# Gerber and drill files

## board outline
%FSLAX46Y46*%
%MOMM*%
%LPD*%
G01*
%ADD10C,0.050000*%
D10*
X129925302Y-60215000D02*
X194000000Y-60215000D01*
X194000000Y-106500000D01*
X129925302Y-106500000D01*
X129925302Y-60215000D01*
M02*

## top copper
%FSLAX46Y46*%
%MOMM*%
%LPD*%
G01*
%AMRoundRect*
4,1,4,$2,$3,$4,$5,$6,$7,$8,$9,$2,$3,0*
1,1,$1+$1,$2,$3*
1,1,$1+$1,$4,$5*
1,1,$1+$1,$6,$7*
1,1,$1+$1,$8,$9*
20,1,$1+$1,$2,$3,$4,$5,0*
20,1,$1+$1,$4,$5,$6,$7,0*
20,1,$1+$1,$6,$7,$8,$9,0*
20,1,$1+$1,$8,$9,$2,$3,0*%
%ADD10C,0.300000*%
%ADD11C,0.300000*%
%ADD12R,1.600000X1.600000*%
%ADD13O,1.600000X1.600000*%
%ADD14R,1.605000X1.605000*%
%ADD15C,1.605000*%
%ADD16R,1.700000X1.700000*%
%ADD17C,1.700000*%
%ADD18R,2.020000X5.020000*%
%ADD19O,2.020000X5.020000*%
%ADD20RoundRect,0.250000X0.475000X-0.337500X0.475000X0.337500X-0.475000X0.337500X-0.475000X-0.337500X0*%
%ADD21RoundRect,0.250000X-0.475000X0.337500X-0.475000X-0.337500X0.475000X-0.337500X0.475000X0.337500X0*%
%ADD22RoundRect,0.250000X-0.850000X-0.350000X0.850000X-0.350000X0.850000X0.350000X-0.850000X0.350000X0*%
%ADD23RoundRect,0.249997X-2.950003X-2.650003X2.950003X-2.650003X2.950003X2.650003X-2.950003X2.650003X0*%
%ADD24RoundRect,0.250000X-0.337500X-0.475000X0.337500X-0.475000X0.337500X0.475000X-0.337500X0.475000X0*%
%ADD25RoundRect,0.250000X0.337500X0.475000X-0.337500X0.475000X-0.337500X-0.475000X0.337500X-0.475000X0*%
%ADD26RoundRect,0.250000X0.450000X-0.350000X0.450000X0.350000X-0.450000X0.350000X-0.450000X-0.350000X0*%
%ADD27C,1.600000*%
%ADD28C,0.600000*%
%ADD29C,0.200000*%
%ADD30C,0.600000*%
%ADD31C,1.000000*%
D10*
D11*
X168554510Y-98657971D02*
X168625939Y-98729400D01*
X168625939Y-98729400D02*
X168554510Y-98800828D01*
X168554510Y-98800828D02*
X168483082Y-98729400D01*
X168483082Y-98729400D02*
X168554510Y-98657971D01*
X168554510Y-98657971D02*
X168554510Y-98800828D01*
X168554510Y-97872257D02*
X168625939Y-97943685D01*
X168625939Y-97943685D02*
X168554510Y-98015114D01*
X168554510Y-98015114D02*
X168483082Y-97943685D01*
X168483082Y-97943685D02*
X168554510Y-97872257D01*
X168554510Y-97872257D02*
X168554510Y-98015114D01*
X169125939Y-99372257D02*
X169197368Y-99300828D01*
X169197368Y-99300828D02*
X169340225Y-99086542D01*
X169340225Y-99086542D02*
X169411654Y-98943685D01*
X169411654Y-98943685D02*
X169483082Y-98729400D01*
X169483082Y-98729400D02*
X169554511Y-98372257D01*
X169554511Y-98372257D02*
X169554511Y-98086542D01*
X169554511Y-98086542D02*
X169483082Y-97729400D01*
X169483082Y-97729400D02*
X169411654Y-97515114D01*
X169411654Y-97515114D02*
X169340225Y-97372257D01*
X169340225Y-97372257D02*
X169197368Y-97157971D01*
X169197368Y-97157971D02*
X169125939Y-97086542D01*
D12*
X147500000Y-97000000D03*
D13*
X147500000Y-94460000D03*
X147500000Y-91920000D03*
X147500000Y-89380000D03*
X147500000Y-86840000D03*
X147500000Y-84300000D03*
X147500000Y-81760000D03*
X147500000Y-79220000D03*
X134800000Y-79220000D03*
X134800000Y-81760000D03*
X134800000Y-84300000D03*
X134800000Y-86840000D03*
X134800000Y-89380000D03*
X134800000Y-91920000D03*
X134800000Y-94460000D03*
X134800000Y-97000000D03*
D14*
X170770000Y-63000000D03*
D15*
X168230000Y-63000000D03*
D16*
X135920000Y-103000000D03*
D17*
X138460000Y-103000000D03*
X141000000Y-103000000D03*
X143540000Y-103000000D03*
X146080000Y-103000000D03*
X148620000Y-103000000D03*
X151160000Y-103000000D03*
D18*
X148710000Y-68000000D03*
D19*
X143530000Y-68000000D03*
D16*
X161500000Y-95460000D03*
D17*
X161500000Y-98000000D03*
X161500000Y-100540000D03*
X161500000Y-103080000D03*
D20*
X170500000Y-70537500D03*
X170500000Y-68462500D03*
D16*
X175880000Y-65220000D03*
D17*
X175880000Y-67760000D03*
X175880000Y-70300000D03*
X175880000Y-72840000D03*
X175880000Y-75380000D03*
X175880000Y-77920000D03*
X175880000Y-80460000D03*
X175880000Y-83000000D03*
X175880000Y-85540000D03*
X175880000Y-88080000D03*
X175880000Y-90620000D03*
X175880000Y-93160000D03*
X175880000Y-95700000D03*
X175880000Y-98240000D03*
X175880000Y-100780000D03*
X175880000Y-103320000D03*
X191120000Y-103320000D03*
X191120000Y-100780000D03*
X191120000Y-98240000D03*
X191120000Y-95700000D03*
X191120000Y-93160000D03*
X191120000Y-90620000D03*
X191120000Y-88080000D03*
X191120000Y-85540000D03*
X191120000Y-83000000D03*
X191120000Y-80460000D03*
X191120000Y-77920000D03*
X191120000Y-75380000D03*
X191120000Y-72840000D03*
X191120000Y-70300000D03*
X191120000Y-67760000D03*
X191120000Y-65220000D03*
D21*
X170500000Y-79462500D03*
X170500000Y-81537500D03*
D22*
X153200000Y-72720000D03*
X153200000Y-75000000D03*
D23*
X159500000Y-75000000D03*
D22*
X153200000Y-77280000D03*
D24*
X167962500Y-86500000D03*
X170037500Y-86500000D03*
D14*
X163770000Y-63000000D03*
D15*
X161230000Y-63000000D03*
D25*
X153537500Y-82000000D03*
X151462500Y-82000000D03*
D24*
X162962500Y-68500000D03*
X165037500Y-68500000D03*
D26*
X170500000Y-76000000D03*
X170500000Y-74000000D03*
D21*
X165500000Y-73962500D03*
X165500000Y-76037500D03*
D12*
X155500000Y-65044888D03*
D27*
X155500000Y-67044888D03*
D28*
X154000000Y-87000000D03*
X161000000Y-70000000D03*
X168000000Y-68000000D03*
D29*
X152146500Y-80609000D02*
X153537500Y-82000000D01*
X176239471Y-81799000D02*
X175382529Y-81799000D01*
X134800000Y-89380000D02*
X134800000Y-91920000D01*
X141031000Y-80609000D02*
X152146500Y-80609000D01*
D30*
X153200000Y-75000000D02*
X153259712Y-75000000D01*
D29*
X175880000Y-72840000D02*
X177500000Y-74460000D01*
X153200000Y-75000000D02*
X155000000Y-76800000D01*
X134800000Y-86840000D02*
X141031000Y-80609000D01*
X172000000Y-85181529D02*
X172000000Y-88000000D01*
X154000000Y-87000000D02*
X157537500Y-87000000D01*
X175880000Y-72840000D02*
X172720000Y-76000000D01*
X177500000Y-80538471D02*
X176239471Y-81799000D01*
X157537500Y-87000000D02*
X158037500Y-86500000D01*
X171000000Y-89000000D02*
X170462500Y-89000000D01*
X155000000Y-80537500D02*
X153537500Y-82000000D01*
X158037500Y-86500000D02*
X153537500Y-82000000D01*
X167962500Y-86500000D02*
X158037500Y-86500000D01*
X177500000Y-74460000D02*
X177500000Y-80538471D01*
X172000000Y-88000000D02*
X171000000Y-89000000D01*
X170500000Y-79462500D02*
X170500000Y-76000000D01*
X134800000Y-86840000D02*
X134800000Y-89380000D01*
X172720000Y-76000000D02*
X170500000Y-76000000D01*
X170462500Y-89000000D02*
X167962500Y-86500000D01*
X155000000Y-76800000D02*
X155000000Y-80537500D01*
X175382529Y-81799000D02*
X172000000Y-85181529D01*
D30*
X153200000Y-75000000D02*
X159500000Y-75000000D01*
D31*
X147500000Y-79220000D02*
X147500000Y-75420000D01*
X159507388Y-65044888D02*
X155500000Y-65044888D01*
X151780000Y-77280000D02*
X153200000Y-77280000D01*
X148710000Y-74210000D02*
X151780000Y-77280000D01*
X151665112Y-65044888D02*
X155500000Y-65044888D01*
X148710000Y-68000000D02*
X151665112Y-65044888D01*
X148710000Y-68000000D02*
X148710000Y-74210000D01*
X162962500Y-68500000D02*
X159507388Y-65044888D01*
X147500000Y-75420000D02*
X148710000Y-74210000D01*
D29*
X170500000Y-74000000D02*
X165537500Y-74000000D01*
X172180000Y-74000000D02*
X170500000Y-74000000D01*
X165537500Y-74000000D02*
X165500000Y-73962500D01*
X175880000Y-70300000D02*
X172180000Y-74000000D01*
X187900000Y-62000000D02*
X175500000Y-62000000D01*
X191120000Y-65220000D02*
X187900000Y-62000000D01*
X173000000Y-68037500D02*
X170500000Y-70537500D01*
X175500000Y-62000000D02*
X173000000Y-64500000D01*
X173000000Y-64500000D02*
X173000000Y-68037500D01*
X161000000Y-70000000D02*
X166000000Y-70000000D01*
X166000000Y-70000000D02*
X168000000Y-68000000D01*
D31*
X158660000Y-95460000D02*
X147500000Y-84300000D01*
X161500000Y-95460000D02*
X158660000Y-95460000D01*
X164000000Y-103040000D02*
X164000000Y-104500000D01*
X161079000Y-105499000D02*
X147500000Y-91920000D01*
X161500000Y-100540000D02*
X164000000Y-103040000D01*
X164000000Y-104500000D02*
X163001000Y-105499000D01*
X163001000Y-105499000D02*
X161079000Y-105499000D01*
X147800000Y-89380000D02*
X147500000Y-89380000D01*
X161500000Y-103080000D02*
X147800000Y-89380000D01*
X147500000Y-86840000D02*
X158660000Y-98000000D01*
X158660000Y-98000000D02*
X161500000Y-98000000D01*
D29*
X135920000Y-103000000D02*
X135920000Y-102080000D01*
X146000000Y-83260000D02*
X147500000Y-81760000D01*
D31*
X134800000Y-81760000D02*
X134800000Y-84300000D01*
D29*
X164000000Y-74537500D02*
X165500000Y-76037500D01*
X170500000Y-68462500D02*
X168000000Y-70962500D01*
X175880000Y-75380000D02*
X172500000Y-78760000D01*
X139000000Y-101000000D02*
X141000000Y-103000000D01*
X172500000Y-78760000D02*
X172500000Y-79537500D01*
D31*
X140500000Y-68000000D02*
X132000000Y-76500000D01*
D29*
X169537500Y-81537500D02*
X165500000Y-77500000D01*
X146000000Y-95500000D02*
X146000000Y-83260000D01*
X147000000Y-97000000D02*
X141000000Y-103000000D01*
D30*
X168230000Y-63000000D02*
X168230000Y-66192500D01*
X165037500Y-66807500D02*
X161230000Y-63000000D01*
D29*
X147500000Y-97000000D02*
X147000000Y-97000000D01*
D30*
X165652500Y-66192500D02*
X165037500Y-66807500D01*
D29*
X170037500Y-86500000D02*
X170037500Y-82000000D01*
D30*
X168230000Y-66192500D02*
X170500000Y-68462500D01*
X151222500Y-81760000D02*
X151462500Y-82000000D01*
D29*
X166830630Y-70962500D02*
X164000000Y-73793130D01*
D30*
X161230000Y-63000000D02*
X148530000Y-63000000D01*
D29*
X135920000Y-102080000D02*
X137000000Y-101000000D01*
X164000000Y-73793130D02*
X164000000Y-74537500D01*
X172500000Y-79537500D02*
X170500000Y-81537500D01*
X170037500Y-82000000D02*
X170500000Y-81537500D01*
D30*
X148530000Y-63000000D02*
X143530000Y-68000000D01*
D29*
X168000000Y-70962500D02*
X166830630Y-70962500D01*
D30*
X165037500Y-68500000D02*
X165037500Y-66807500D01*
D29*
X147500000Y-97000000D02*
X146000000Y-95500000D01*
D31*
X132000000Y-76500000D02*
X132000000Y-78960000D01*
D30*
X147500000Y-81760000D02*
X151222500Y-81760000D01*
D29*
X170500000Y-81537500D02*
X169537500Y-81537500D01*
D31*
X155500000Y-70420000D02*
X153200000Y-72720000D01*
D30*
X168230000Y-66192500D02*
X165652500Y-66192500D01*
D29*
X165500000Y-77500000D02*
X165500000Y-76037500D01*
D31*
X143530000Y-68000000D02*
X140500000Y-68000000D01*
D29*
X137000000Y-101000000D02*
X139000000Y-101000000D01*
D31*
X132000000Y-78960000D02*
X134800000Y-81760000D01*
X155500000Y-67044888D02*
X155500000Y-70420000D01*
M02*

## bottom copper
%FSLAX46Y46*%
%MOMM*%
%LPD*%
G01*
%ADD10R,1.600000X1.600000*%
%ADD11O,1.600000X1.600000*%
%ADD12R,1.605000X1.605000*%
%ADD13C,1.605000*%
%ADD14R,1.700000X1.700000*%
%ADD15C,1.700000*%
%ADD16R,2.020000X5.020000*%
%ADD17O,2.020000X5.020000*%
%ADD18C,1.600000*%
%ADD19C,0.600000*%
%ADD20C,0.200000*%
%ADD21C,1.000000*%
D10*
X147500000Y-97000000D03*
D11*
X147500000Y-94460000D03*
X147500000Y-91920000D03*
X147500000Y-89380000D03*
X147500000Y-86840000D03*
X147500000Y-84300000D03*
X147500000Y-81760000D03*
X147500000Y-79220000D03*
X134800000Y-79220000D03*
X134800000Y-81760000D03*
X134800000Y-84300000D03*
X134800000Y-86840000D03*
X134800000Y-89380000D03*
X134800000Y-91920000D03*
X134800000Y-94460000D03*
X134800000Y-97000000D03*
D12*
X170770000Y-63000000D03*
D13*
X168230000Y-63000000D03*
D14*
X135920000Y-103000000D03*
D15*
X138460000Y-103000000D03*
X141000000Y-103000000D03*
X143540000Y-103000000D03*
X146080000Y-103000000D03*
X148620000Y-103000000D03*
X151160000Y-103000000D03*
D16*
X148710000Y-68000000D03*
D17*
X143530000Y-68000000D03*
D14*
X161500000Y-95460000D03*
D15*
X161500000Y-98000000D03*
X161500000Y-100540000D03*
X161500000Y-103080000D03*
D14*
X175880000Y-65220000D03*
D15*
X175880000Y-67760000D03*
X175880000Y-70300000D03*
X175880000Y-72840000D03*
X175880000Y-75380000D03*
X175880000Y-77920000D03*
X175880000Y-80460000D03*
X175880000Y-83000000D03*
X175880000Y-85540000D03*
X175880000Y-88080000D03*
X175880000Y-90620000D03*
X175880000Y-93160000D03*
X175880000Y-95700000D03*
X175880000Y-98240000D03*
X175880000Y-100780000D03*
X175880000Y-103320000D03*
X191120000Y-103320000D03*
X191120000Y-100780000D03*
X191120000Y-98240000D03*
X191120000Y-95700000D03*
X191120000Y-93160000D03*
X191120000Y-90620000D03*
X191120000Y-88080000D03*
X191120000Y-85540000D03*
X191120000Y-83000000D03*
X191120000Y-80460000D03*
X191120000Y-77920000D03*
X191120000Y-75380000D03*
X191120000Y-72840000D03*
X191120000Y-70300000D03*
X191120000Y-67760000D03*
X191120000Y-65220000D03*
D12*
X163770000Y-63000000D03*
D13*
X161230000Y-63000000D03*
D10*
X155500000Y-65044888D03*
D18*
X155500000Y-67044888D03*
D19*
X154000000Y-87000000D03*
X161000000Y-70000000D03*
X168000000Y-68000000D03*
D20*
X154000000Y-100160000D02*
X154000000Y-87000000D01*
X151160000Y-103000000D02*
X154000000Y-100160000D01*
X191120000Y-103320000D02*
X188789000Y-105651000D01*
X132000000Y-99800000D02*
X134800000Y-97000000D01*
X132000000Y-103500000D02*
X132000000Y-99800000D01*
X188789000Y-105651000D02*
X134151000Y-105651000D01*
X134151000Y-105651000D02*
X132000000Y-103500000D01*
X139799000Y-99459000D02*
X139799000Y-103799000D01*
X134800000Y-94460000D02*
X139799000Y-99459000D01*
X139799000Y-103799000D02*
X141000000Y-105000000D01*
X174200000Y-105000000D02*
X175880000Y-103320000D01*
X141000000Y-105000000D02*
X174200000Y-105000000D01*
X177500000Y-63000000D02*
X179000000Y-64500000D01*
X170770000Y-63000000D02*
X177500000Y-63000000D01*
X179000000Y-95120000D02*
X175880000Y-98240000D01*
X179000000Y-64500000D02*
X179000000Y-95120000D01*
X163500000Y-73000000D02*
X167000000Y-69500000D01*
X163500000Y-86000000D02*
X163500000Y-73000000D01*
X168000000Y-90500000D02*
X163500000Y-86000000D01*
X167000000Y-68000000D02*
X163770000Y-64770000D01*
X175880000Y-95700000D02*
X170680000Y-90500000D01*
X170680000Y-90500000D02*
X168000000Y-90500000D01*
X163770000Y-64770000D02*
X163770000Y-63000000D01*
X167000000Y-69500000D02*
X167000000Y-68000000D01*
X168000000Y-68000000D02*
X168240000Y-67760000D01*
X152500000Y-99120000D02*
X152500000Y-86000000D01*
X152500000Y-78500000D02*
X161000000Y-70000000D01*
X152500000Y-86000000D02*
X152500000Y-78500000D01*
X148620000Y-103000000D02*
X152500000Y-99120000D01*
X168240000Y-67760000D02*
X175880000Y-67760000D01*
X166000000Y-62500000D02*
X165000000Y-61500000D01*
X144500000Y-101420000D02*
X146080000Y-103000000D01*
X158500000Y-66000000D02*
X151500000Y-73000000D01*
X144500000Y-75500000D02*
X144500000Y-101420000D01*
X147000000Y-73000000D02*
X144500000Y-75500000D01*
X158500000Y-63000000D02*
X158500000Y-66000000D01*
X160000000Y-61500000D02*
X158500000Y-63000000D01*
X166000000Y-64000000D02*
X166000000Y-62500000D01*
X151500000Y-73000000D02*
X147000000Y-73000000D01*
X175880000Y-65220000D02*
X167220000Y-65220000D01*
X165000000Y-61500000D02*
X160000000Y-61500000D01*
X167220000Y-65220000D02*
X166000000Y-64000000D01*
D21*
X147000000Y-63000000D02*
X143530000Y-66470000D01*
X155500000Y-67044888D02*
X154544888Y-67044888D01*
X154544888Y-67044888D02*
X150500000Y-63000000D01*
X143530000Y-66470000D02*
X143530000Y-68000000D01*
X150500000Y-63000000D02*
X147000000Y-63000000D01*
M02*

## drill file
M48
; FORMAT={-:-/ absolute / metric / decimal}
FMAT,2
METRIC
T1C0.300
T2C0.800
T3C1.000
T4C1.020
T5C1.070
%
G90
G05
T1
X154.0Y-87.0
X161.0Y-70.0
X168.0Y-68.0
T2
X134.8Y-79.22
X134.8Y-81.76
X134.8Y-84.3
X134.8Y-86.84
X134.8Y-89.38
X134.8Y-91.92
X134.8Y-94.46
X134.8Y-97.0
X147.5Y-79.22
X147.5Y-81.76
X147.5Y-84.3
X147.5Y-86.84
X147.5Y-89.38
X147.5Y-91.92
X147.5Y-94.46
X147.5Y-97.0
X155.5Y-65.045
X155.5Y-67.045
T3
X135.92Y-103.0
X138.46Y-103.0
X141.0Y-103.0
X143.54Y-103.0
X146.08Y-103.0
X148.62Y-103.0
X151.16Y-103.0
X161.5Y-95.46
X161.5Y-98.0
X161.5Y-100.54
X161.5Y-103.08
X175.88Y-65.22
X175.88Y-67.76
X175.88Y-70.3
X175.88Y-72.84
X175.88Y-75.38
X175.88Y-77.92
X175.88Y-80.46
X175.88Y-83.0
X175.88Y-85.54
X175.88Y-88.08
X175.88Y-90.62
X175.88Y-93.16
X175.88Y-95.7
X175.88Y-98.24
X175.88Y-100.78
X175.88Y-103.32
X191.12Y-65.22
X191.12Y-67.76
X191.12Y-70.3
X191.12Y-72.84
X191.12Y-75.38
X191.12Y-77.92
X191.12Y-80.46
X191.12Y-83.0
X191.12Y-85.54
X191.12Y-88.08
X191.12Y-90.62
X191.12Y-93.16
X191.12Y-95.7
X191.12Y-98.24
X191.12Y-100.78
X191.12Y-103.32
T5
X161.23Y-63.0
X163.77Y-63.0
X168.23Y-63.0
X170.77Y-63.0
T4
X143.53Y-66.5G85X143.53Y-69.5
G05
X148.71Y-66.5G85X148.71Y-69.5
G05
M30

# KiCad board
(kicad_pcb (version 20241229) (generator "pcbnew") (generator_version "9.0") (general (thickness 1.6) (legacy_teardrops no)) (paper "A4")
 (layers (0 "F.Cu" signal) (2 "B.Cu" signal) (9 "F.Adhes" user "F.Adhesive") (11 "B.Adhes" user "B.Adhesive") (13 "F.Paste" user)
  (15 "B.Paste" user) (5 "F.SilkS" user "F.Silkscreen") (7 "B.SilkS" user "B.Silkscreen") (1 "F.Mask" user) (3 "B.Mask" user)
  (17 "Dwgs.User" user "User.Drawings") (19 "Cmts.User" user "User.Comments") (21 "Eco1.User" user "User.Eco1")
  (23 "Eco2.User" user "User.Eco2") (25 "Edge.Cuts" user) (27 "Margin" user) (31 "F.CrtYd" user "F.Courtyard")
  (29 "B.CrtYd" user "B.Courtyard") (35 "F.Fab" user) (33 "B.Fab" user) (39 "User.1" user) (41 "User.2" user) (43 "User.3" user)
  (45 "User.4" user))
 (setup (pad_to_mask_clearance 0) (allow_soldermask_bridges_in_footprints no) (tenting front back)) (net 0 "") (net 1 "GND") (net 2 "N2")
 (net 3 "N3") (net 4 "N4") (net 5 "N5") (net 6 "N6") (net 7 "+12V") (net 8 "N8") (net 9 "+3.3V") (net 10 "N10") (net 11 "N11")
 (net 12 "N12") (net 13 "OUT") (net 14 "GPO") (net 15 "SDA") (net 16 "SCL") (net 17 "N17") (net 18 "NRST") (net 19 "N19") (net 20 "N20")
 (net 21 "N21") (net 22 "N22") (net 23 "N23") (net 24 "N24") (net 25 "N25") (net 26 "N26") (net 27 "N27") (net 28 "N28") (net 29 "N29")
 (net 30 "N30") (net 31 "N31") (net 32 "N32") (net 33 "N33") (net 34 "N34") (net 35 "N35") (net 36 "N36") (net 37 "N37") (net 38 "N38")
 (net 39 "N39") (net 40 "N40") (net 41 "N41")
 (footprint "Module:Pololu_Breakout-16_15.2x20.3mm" (layer "F.Cu") (at 147.5 97 180)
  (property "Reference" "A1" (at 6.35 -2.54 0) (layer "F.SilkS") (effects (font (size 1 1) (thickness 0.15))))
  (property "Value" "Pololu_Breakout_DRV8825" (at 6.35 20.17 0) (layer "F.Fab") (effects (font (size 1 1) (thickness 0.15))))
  (pad "1" thru_hole rect (at 0 0 180) (size 1.6 1.6) (drill 0.8) (layers "*.Cu" "*.Mask") (remove_unused_layers no) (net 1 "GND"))
  (pad "2" thru_hole oval (at 0 2.54 180) (size 1.6 1.6) (drill 0.8) (layers "*.Cu" "*.Mask") (remove_unused_layers no) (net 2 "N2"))
  (pad "3" thru_hole oval (at 0 5.08 180) (size 1.6 1.6) (drill 0.8) (layers "*.Cu" "*.Mask") (remove_unused_layers no) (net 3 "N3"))
  (pad "4" thru_hole oval (at 0 7.62 180) (size 1.6 1.6) (drill 0.8) (layers "*.Cu" "*.Mask") (remove_unused_layers no) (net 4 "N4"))
  (pad "5" thru_hole oval (at 0 10.16 180) (size 1.6 1.6) (drill 0.8) (layers "*.Cu" "*.Mask") (remove_unused_layers no) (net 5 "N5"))
  (pad "6" thru_hole oval (at 0 12.7 180) (size 1.6 1.6) (drill 0.8) (layers "*.Cu" "*.Mask") (remove_unused_layers no) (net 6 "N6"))
  (pad "7" thru_hole oval (at 0 15.24 180) (size 1.6 1.6) (drill 0.8) (layers "*.Cu" "*.Mask") (remove_unused_layers no) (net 1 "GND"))
  (pad "8" thru_hole oval (at 0 17.78 180) (size 1.6 1.6) (drill 0.8) (layers "*.Cu" "*.Mask") (remove_unused_layers no) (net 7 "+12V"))
  (pad "9" thru_hole oval (at 12.7 17.78 180) (size 1.6 1.6) (drill 0.8) (layers "*.Cu" "*.Mask") (remove_unused_layers no) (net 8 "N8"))
  (pad "10" thru_hole oval (at 12.7 15.24 180) (size 1.6 1.6) (drill 0.8) (layers "*.Cu" "*.Mask") (remove_unused_layers no) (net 1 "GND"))
  (pad "11" thru_hole oval (at 12.7 12.7 180) (size 1.6 1.6) (drill 0.8) (layers "*.Cu" "*.Mask") (remove_unused_layers no) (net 1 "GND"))
  (pad "12" thru_hole oval (at 12.7 10.16 180) (size 1.6 1.6) (drill 0.8) (layers "*.Cu" "*.Mask") (remove_unused_layers no) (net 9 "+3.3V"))
  (pad "13" thru_hole oval (at 12.7 7.62 180) (size 1.6 1.6) (drill 0.8) (layers "*.Cu" "*.Mask") (remove_unused_layers no) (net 9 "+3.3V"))
  (pad "14" thru_hole oval (at 12.7 5.08 180) (size 1.6 1.6) (drill 0.8) (layers "*.Cu" "*.Mask") (remove_unused_layers no) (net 9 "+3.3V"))
  (pad "15" thru_hole oval (at 12.7 2.54 180) (size 1.6 1.6) (drill 0.8) (layers "*.Cu" "*.Mask") (remove_unused_layers no) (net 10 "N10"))
  (pad "16" thru_hole oval (at 12.7 0 180) (size 1.6 1.6) (drill 0.8) (layers "*.Cu" "*.Mask") (remove_unused_layers no) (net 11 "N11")))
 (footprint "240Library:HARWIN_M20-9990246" (layer "F.Cu") (at 169.5 63 180)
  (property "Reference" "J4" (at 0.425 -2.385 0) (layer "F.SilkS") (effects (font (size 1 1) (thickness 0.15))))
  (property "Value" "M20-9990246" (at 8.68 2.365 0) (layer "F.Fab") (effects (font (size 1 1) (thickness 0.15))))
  (pad "1" thru_hole rect (at -1.27 0 180) (size 1.605 1.605) (drill 1.07) (layers "*.Cu" "*.Mask") (remove_unused_layers no) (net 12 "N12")
   (solder_mask_margin 0.102))
  (pad "2" thru_hole circle (at 1.27 0 180) (size 1.605 1.605) (drill 1.07) (layers "*.Cu" "*.Mask") (remove_unused_layers no) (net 1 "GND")
   (solder_mask_margin 0.102)))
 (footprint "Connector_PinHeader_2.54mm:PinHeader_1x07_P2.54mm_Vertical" (layer "F.Cu") (at 135.92 103 90)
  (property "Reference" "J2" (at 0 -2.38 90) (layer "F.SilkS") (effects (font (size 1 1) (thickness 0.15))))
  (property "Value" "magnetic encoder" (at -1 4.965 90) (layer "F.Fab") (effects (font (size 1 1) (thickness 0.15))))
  (pad "1" thru_hole rect (at 0 0 90) (size 1.7 1.7) (drill 1) (layers "*.Cu" "*.Mask") (remove_unused_layers no) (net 1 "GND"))
  (pad "2" thru_hole circle (at 0 2.54 90) (size 1.7 1.7) (drill 1) (layers "*.Cu" "*.Mask") (remove_unused_layers no) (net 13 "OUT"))
  (pad "3" thru_hole circle (at 0 5.08 90) (size 1.7 1.7) (drill 1) (layers "*.Cu" "*.Mask") (remove_unused_layers no) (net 1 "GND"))
  (pad "4" thru_hole circle (at 0 7.62 90) (size 1.7 1.7) (drill 1) (layers "*.Cu" "*.Mask") (remove_unused_layers no) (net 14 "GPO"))
  (pad "5" thru_hole circle (at 0 10.16 90) (size 1.7 1.7) (drill 1) (layers "*.Cu" "*.Mask") (remove_unused_layers no) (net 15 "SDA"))
  (pad "6" thru_hole circle (at 0 12.7 90) (size 1.7 1.7) (drill 1) (layers "*.Cu" "*.Mask") (remove_unused_layers no) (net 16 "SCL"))
  (pad "7" thru_hole circle (at 0 15.24 90) (size 1.7 1.7) (drill 1) (layers "*.Cu" "*.Mask") (remove_unused_layers no) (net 9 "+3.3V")))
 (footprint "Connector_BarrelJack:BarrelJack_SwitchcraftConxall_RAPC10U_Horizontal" (layer "F.Cu") (at 148.71 68)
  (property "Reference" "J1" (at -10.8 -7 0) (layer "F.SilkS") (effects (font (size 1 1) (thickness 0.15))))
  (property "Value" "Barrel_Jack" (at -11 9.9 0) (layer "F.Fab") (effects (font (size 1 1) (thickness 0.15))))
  (pad "1" thru_hole rect (at 0 0) (size 2.02 5.02) (drill oval 1.02 4.02) (layers "*.Cu" "*.Mask") (remove_unused_layers no) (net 7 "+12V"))
  (pad "2" thru_hole oval (at -5.18 0) (size 2.02 5.02) (drill oval 1.02 4.02) (layers "*.Cu" "*.Mask") (remove_unused_layers no)
   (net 1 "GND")))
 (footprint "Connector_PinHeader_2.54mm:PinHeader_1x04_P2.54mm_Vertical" (layer "F.Cu") (at 161.5 95.46)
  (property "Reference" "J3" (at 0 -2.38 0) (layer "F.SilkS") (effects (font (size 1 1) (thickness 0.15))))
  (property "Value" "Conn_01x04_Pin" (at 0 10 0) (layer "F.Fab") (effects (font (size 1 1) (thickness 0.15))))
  (pad "1" thru_hole rect (at 0 0) (size 1.7 1.7) (drill 1) (layers "*.Cu" "*.Mask") (remove_unused_layers no) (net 6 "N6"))
  (pad "2" thru_hole circle (at 0 2.54) (size 1.7 1.7) (drill 1) (layers "*.Cu" "*.Mask") (remove_unused_layers no) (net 5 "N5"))
  (pad "3" thru_hole circle (at 0 5.08) (size 1.7 1.7) (drill 1) (layers "*.Cu" "*.Mask") (remove_unused_layers no) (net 3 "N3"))
  (pad "4" thru_hole circle (at 0 7.62) (size 1.7 1.7) (drill 1) (layers "*.Cu" "*.Mask") (remove_unused_layers no) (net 4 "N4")))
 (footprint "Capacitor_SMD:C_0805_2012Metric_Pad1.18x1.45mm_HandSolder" (layer "F.Cu") (at 170.5 69.5 90)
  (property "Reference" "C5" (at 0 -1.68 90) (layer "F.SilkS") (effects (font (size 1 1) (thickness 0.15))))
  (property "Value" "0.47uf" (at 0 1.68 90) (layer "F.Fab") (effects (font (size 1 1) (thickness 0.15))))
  (pad "1" smd roundrect (at -1.0375 0 90) (size 1.175 1.45) (layers "F.Cu" "F.Mask" "F.Paste") (roundrect_rratio 0.212766) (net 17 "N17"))
  (pad "2" smd roundrect (at 1.0375 0 90) (size 1.175 1.45) (layers "F.Cu" "F.Mask" "F.Paste") (roundrect_rratio 0.212766) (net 1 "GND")))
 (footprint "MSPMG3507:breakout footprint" (layer "F.Cu") (at 182.73 84.78)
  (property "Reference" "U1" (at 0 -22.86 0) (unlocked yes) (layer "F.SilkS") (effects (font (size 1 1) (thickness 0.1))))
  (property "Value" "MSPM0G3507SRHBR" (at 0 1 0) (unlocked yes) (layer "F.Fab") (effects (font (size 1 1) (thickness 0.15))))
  (pad "1" thru_hole rect (at -6.85 -19.56) (size 1.7 1.7) (drill 1) (layers "*.Cu" "*.Mask") (remove_unused_layers no) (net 15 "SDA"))
  (pad "2" thru_hole circle (at -6.85 -17.02) (size 1.7 1.7) (drill 1) (layers "*.Cu" "*.Mask") (remove_unused_layers no) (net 16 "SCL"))
  (pad "3" thru_hole circle (at -6.85 -14.48) (size 1.7 1.7) (drill 1) (layers "*.Cu" "*.Mask") (remove_unused_layers no) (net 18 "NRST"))
  (pad "4" thru_hole circle (at -6.85 -11.94) (size 1.7 1.7) (drill 1) (layers "*.Cu" "*.Mask") (remove_unused_layers no) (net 9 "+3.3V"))
  (pad "5" thru_hole circle (at -6.85 -9.4) (size 1.7 1.7) (drill 1) (layers "*.Cu" "*.Mask") (remove_unused_layers no) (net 1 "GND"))
  (pad "6" thru_hole circle (at -6.85 -6.86) (size 1.7 1.7) (drill 1) (layers "*.Cu" "*.Mask") (remove_unused_layers no) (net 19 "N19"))
  (pad "7" thru_hole circle (at -6.85 -4.32) (size 1.7 1.7) (drill 1) (layers "*.Cu" "*.Mask") (remove_unused_layers no) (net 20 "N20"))
  (pad "8" thru_hole circle (at -6.85 -1.78) (size 1.7 1.7) (drill 1) (layers "*.Cu" "*.Mask") (remove_unused_layers no) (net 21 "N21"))
  (pad "9" thru_hole circle (at -6.85 0.76) (size 1.7 1.7) (drill 1) (layers "*.Cu" "*.Mask") (remove_unused_layers no) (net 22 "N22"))
  (pad "10" thru_hole circle (at -6.85 3.3) (size 1.7 1.7) (drill 1) (layers "*.Cu" "*.Mask") (remove_unused_layers no) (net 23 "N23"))
  (pad "11" thru_hole circle (at -6.85 5.84) (size 1.7 1.7) (drill 1) (layers "*.Cu" "*.Mask") (remove_unused_layers no) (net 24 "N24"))
  (pad "12" thru_hole circle (at -6.85 8.38) (size 1.7 1.7) (drill 1) (layers "*.Cu" "*.Mask") (remove_unused_layers no) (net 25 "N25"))
  (pad "13" thru_hole circle (at -6.85 10.92) (size 1.7 1.7) (drill 1) (layers "*.Cu" "*.Mask") (remove_unused_layers no) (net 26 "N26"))
  (pad "14" thru_hole circle (at -6.85 13.46) (size 1.7 1.7) (drill 1) (layers "*.Cu" "*.Mask") (remove_unused_layers no) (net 12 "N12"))
  (pad "15" thru_hole circle (at -6.85 16) (size 1.7 1.7) (drill 1) (layers "*.Cu" "*.Mask") (remove_unused_layers no) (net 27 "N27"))
  (pad "16" thru_hole circle (at -6.85 18.54) (size 1.7 1.7) (drill 1) (layers "*.Cu" "*.Mask") (remove_unused_layers no) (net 10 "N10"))
  (pad "17" thru_hole circle (at 8.39 18.54) (size 1.7 1.7) (drill 1) (layers "*.Cu" "*.Mask") (remove_unused_layers no) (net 11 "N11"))
  (pad "18" thru_hole circle (at 8.39 16) (size 1.7 1.7) (drill 1) (layers "*.Cu" "*.Mask") (remove_unused_layers no) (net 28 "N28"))
  (pad "19" thru_hole circle (at 8.39 13.46) (size 1.7 1.7) (drill 1) (layers "*.Cu" "*.Mask") (remove_unused_layers no) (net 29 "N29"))
  (pad "20" thru_hole circle (at 8.39 10.92) (size 1.7 1.7) (drill 1) (layers "*.Cu" "*.Mask") (remove_unused_layers no) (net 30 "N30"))
  (pad "21" thru_hole circle (at 8.39 8.38) (size 1.7 1.7) (drill 1) (layers "*.Cu" "*.Mask") (remove_unused_layers no) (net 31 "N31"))
  (pad "22" thru_hole circle (at 8.39 5.84) (size 1.7 1.7) (drill 1) (layers "*.Cu" "*.Mask") (remove_unused_layers no) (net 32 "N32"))
  (pad "23" thru_hole circle (at 8.39 3.3) (size 1.7 1.7) (drill 1) (layers "*.Cu" "*.Mask") (remove_unused_layers no) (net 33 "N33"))
  (pad "24" thru_hole circle (at 8.39 0.76) (size 1.7 1.7) (drill 1) (layers "*.Cu" "*.Mask") (remove_unused_layers no) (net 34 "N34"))
  (pad "25" thru_hole circle (at 8.39 -1.78) (size 1.7 1.7) (drill 1) (layers "*.Cu" "*.Mask") (remove_unused_layers no) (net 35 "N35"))
  (pad "26" thru_hole circle (at 8.39 -4.32) (size 1.7 1.7) (drill 1) (layers "*.Cu" "*.Mask") (remove_unused_layers no) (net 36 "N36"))
  (pad "27" thru_hole circle (at 8.39 -6.86) (size 1.7 1.7) (drill 1) (layers "*.Cu" "*.Mask") (remove_unused_layers no) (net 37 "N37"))
  (pad "28" thru_hole circle (at 8.39 -9.4) (size 1.7 1.7) (drill 1) (layers "*.Cu" "*.Mask") (remove_unused_layers no) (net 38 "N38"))
  (pad "29" thru_hole circle (at 8.39 -11.94) (size 1.7 1.7) (drill 1) (layers "*.Cu" "*.Mask") (remove_unused_layers no) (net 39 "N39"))
  (pad "30" thru_hole circle (at 8.39 -14.48) (size 1.7 1.7) (drill 1) (layers "*.Cu" "*.Mask") (remove_unused_layers no) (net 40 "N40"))
  (pad "31" thru_hole circle (at 8.39 -17.02) (size 1.7 1.7) (drill 1) (layers "*.Cu" "*.Mask") (remove_unused_layers no) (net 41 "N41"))
  (pad "32" thru_hole circle (at 8.39 -19.56) (size 1.7 1.7) (drill 1) (layers "*.Cu" "*.Mask") (remove_unused_layers no) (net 17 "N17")))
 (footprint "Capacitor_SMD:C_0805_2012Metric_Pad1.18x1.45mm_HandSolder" (layer "F.Cu") (at 170.5 80.5 -90)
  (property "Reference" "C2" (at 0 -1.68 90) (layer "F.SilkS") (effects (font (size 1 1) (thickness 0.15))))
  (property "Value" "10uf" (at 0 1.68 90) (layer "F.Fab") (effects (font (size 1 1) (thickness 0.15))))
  (pad "1" smd roundrect (at -1.0375 0 270) (size 1.175 1.45) (layers "F.Cu" "F.Mask" "F.Paste") (roundrect_rratio 0.212766) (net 9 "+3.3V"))
  (pad "2" smd roundrect (at 1.0375 0 270) (size 1.175 1.45) (layers "F.Cu" "F.Mask" "F.Paste") (roundrect_rratio 0.212766) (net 1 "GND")))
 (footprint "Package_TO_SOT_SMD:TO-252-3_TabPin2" (layer "F.Cu") (at 158.24 75)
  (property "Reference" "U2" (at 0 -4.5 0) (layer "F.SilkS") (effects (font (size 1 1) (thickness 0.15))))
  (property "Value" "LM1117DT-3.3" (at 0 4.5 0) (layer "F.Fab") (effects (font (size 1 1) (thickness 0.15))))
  (pad "" smd roundrect (at -0.415 -1.525) (size 3.05 2.75) (layers "F.Paste") (roundrect_rratio 0.090909))
  (pad "" smd roundrect (at -0.415 1.525) (size 3.05 2.75) (layers "F.Paste") (roundrect_rratio 0.090909))
  (pad "" smd roundrect (at 2.935 -1.525) (size 3.05 2.75) (layers "F.Paste") (roundrect_rratio 0.090909))
  (pad "" smd roundrect (at 2.935 1.525) (size 3.05 2.75) (layers "F.Paste") (roundrect_rratio 0.090909))
  (pad "1" smd roundrect (at -5.04 -2.28) (size 2.2 1.2) (layers "F.Cu" "F.Mask" "F.Paste") (roundrect_rratio 0.208333) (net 1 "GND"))
  (pad "2" smd roundrect (at -5.04 0) (size 2.2 1.2) (layers "F.Cu" "F.Mask" "F.Paste") (roundrect_rratio 0.208333) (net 9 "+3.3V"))
  (pad "2" smd roundrect (at 1.26 0) (size 6.4 5.8) (layers "F.Cu" "F.Mask") (roundrect_rratio 0.043103) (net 9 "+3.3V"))
  (pad "3" smd roundrect (at -5.04 2.28) (size 2.2 1.2) (layers "F.Cu" "F.Mask" "F.Paste") (roundrect_rratio 0.208333) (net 7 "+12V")))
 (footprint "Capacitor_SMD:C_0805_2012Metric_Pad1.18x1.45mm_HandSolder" (layer "F.Cu") (at 169 86.5)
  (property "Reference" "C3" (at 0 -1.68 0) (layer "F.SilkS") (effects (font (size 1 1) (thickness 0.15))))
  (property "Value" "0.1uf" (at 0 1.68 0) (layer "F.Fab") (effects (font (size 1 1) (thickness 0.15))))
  (pad "1" smd roundrect (at -1.0375 0) (size 1.175 1.45) (layers "F.Cu" "F.Mask" "F.Paste") (roundrect_rratio 0.212766) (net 9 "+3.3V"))
  (pad "2" smd roundrect (at 1.0375 0) (size 1.175 1.45) (layers "F.Cu" "F.Mask" "F.Paste") (roundrect_rratio 0.212766) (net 1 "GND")))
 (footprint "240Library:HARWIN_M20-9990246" (layer "F.Cu") (at 162.5 63 180)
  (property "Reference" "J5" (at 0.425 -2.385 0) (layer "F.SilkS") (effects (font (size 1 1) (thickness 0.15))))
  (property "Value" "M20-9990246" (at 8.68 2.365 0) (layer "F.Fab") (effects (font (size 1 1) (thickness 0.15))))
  (pad "1" thru_hole rect (at -1.27 0 180) (size 1.605 1.605) (drill 1.07) (layers "*.Cu" "*.Mask") (remove_unused_layers no) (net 26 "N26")
   (solder_mask_margin 0.102))
  (pad "2" thru_hole circle (at 1.27 0 180) (size 1.605 1.605) (drill 1.07) (layers "*.Cu" "*.Mask") (remove_unused_layers no) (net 1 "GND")
   (solder_mask_margin 0.102)))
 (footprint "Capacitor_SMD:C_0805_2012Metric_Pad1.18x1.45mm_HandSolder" (layer "F.Cu") (at 152.5 82 180)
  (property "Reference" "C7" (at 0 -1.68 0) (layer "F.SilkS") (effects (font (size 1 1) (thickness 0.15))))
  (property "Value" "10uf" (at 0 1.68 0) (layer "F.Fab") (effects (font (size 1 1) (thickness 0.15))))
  (pad "1" smd roundrect (at -1.0375 0 180) (size 1.175 1.45) (layers "F.Cu" "F.Mask" "F.Paste") (roundrect_rratio 0.212766) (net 9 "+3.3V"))
  (pad "2" smd roundrect (at 1.0375 0 180) (size 1.175 1.45) (layers "F.Cu" "F.Mask" "F.Paste") (roundrect_rratio 0.212766) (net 1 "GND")))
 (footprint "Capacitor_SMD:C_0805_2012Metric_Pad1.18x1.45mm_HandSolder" (layer "F.Cu") (at 164 68.5)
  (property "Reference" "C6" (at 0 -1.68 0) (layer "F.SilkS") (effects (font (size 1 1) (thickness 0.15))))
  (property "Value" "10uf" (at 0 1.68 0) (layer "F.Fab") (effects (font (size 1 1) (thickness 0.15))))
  (pad "1" smd roundrect (at -1.0375 0) (size 1.175 1.45) (layers "F.Cu" "F.Mask" "F.Paste") (roundrect_rratio 0.212766) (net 7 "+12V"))
  (pad "2" smd roundrect (at 1.0375 0) (size 1.175 1.45) (layers "F.Cu" "F.Mask" "F.Paste") (roundrect_rratio 0.212766) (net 1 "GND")))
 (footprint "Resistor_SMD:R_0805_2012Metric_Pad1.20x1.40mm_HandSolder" (layer "F.Cu") (at 170.5 75 90)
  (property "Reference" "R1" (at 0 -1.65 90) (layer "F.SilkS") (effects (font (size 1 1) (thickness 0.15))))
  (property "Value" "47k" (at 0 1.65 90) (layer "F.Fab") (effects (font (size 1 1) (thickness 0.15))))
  (pad "1" smd roundrect (at -1 0 90) (size 1.2 1.4) (layers "F.Cu" "F.Mask" "F.Paste") (roundrect_rratio 0.208333) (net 9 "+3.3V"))
  (pad "2" smd roundrect (at 1 0 90) (size 1.2 1.4) (layers "F.Cu" "F.Mask" "F.Paste") (roundrect_rratio 0.208333) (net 18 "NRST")))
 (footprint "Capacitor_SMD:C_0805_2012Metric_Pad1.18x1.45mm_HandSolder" (layer "F.Cu") (at 165.5 75 -90)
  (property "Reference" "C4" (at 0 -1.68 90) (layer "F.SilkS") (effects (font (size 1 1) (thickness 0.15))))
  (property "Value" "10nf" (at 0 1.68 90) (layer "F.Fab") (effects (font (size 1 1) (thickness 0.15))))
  (pad "1" smd roundrect (at -1.0375 0 270) (size 1.175 1.45) (layers "F.Cu" "F.Mask" "F.Paste") (roundrect_rratio 0.212766) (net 18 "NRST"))
  (pad "2" smd roundrect (at 1.0375 0 270) (size 1.175 1.45) (layers "F.Cu" "F.Mask" "F.Paste") (roundrect_rratio 0.212766) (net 1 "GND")))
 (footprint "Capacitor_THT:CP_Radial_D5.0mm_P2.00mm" (layer "F.Cu") (at 155.5 65.044888 -90)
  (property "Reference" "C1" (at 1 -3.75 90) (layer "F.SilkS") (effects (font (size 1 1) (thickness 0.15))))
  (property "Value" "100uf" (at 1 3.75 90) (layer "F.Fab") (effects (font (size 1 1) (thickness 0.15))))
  (pad "1" thru_hole rect (at 0 0 270) (size 1.6 1.6) (drill 0.8) (layers "*.Cu" "*.Mask") (remove_unused_layers no) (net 7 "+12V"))
  (pad "2" thru_hole circle (at 2 0 270) (size 1.6 1.6) (drill 0.8) (layers "*.Cu" "*.Mask") (remove_unused_layers no) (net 1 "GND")))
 (gr_rect (start 129.925302 60.215) (end 194 106.5) (stroke (width 0.05) (type default)) (fill no) (layer "Edge.Cuts"))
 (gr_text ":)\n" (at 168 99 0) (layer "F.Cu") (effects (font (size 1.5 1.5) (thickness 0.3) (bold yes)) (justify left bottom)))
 (segment (start 152.1465 80.609) (end 153.5375 82) (width 0.2) (layer "F.Cu") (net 9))
 (segment (start 176.239471 81.799) (end 175.382529 81.799) (width 0.2) (layer "F.Cu") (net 9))
 (segment (start 134.8 89.38) (end 134.8 91.92) (width 0.2) (layer "F.Cu") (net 9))
 (segment (start 141.031 80.609) (end 152.1465 80.609) (width 0.2) (layer "F.Cu") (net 9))
 (segment (start 153.2 75) (end 153.259712 75) (width 0.6) (layer "F.Cu") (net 9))
 (segment (start 175.88 72.84) (end 177.5 74.46) (width 0.2) (layer "F.Cu") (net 9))
 (segment (start 153.2 75) (end 155 76.8) (width 0.2) (layer "F.Cu") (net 9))
 (segment (start 134.8 86.84) (end 141.031 80.609) (width 0.2) (layer "F.Cu") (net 9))
 (segment (start 172 85.181529) (end 172 88) (width 0.2) (layer "F.Cu") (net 9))
 (segment (start 154 87) (end 157.5375 87) (width 0.2) (layer "F.Cu") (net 9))
 (segment (start 175.88 72.84) (end 172.72 76) (width 0.2) (layer "F.Cu") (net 9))
 (segment (start 177.5 80.538471) (end 176.239471 81.799) (width 0.2) (layer "F.Cu") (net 9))
 (segment (start 157.5375 87) (end 158.0375 86.5) (width 0.2) (layer "F.Cu") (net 9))
 (segment (start 171 89) (end 170.4625 89) (width 0.2) (layer "F.Cu") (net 9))
 (segment (start 155 80.5375) (end 153.5375 82) (width 0.2) (layer "F.Cu") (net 9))
 (segment (start 158.0375 86.5) (end 153.5375 82) (width 0.2) (layer "F.Cu") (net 9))
 (segment (start 167.9625 86.5) (end 158.0375 86.5) (width 0.2) (layer "F.Cu") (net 9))
 (segment (start 177.5 74.46) (end 177.5 80.538471) (width 0.2) (layer "F.Cu") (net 9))
 (segment (start 172 88) (end 171 89) (width 0.2) (layer "F.Cu") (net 9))
 (segment (start 170.5 79.4625) (end 170.5 76) (width 0.2) (layer "F.Cu") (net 9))
 (segment (start 134.8 86.84) (end 134.8 89.38) (width 0.2) (layer "F.Cu") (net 9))
 (segment (start 172.72 76) (end 170.5 76) (width 0.2) (layer "F.Cu") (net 9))
 (segment (start 170.4625 89) (end 167.9625 86.5) (width 0.2) (layer "F.Cu") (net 9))
 (segment (start 155 76.8) (end 155 80.5375) (width 0.2) (layer "F.Cu") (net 9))
 (segment (start 175.382529 81.799) (end 172 85.181529) (width 0.2) (layer "F.Cu") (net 9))
 (segment (start 153.2 75) (end 159.5 75) (width 0.6) (layer "F.Cu") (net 9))
 (via (at 154 87) (size 0.6) (drill 0.3) (layers "F.Cu" "B.Cu") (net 9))
 (segment (start 154 100.16) (end 154 87) (width 0.2) (layer "B.Cu") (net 9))
 (segment (start 151.16 103) (end 154 100.16) (width 0.2) (layer "B.Cu") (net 9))
 (segment (start 191.12 103.32) (end 188.789 105.651) (width 0.2) (layer "B.Cu") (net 11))
 (segment (start 132 99.8) (end 134.8 97) (width 0.2) (layer "B.Cu") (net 11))
 (segment (start 132 103.5) (end 132 99.8) (width 0.2) (layer "B.Cu") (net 11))
 (segment (start 188.789 105.651) (end 134.151 105.651) (width 0.2) (layer "B.Cu") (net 11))
 (segment (start 134.151 105.651) (end 132 103.5) (width 0.2) (layer "B.Cu") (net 11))
 (segment (start 147.5 79.22) (end 147.5 75.42) (width 1) (layer "F.Cu") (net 7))
 (segment (start 159.507388 65.044888) (end 155.5 65.044888) (width 1) (layer "F.Cu") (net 7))
 (segment (start 151.78 77.28) (end 153.2 77.28) (width 1) (layer "F.Cu") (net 7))
 (segment (start 148.71 74.21) (end 151.78 77.28) (width 1) (layer "F.Cu") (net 7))
 (segment (start 151.665112 65.044888) (end 155.5 65.044888) (width 1) (layer "F.Cu") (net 7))
 (segment (start 148.71 68) (end 151.665112 65.044888) (width 1) (layer "F.Cu") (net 7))
 (segment (start 148.71 68) (end 148.71 74.21) (width 1) (layer "F.Cu") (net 7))
 (segment (start 162.9625 68.5) (end 159.507388 65.044888) (width 1) (layer "F.Cu") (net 7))
 (segment (start 147.5 75.42) (end 148.71 74.21) (width 1) (layer "F.Cu") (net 7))
 (segment (start 139.799 99.459) (end 139.799 103.799) (width 0.2) (layer "B.Cu") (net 10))
 (segment (start 134.8 94.46) (end 139.799 99.459) (width 0.2) (layer "B.Cu") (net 10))
 (segment (start 139.799 103.799) (end 141 105) (width 0.2) (layer "B.Cu") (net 10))
 (segment (start 174.2 105) (end 175.88 103.32) (width 0.2) (layer "B.Cu") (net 10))
 (segment (start 141 105) (end 174.2 105) (width 0.2) (layer "B.Cu") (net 10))
 (segment (start 170.5 74) (end 165.5375 74) (width 0.2) (layer "F.Cu") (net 18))
 (segment (start 172.18 74) (end 170.5 74) (width 0.2) (layer "F.Cu") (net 18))
 (segment (start 165.5375 74) (end 165.5 73.9625) (width 0.2) (layer "F.Cu") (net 18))
 (segment (start 175.88 70.3) (end 172.18 74) (width 0.2) (layer "F.Cu") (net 18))
 (segment (start 187.9 62) (end 175.5 62) (width 0.2) (layer "F.Cu") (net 17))
 (segment (start 191.12 65.22) (end 187.9 62) (width 0.2) (layer "F.Cu") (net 17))
 (segment (start 173 68.0375) (end 170.5 70.5375) (width 0.2) (layer "F.Cu") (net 17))
 (segment (start 175.5 62) (end 173 64.5) (width 0.2) (layer "F.Cu") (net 17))
 (segment (start 173 64.5) (end 173 68.0375) (width 0.2) (layer "F.Cu") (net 17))
 (segment (start 177.5 63) (end 179 64.5) (width 0.2) (layer "B.Cu") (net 12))
 (segment (start 170.77 63) (end 177.5 63) (width 0.2) (layer "B.Cu") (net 12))
 (segment (start 179 95.12) (end 175.88 98.24) (width 0.2) (layer "B.Cu") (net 12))
 (segment (start 179 64.5) (end 179 95.12) (width 0.2) (layer "B.Cu") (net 12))
 (segment (start 163.5 73) (end 167 69.5) (width 0.2) (layer "B.Cu") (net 26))
 (segment (start 163.5 86) (end 163.5 73) (width 0.2) (layer "B.Cu") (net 26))
 (segment (start 168 90.5) (end 163.5 86) (width 0.2) (layer "B.Cu") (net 26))
 (segment (start 167 68) (end 163.77 64.77) (width 0.2) (layer "B.Cu") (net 26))
 (segment (start 175.88 95.7) (end 170.68 90.5) (width 0.2) (layer "B.Cu") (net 26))
 (segment (start 170.68 90.5) (end 168 90.5) (width 0.2) (layer "B.Cu") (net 26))
 (segment (start 163.77 64.77) (end 163.77 63) (width 0.2) (layer "B.Cu") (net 26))
 (segment (start 167 69.5) (end 167 68) (width 0.2) (layer "B.Cu") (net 26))
 (segment (start 161 70) (end 166 70) (width 0.2) (layer "F.Cu") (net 16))
 (segment (start 166 70) (end 168 68) (width 0.2) (layer "F.Cu") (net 16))
 (via (at 161 70) (size 0.6) (drill 0.3) (layers "F.Cu" "B.Cu") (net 16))
 (via (at 168 68) (size 0.6) (drill 0.3) (layers "F.Cu" "B.Cu") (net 16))
 (segment (start 168 68) (end 168.24 67.76) (width 0.2) (layer "B.Cu") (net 16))
 (segment (start 152.5 99.12) (end 152.5 86) (width 0.2) (layer "B.Cu") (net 16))
 (segment (start 152.5 78.5) (end 161 70) (width 0.2) (layer "B.Cu") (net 16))
 (segment (start 152.5 86) (end 152.5 78.5) (width 0.2) (layer "B.Cu") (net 16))
 (segment (start 148.62 103) (end 152.5 99.12) (width 0.2) (layer "B.Cu") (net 16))
 (segment (start 168.24 67.76) (end 175.88 67.76) (width 0.2) (layer "B.Cu") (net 16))
 (segment (start 166 62.5) (end 165 61.5) (width 0.2) (layer "B.Cu") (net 15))
 (segment (start 144.5 101.42) (end 146.08 103) (width 0.2) (layer "B.Cu") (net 15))
 (segment (start 158.5 66) (end 151.5 73) (width 0.2) (layer "B.Cu") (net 15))
 (segment (start 144.5 75.5) (end 144.5 101.42) (width 0.2) (layer "B.Cu") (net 15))
 (segment (start 147 73) (end 144.5 75.5) (width 0.2) (layer "B.Cu") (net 15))
 (segment (start 158.5 63) (end 158.5 66) (width 0.2) (layer "B.Cu") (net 15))
 (segment (start 160 61.5) (end 158.5 63) (width 0.2) (layer "B.Cu") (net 15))
 (segment (start 166 64) (end 166 62.5) (width 0.2) (layer "B.Cu") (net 15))
 (segment (start 151.5 73) (end 147 73) (width 0.2) (layer "B.Cu") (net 15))
 (segment (start 175.88 65.22) (end 167.22 65.22) (width 0.2) (layer "B.Cu") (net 15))
 (segment (start 165 61.5) (end 160 61.5) (width 0.2) (layer "B.Cu") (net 15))
 (segment (start 167.22 65.22) (end 166 64) (width 0.2) (layer "B.Cu") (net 15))
 (segment (start 158.66 95.46) (end 147.5 84.3) (width 1) (layer "F.Cu") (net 6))
 (segment (start 161.5 95.46) (end 158.66 95.46) (width 1) (layer "F.Cu") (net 6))
 (segment (start 164 103.04) (end 164 104.5) (width 1) (layer "F.Cu") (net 3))
 (segment (start 161.079 105.499) (end 147.5 91.92) (width 1) (layer "F.Cu") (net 3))
 (segment (start 161.5 100.54) (end 164 103.04) (width 1) (layer "F.Cu") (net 3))
 (segment (start 164 104.5) (end 163.001 105.499) (width 1) (layer "F.Cu") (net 3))
 (segment (start 163.001 105.499) (end 161.079 105.499) (width 1) (layer "F.Cu") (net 3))
 (segment (start 147.8 89.38) (end 147.5 89.38) (width 1) (layer "F.Cu") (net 4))
 (segment (start 161.5 103.08) (end 147.8 89.38) (width 1) (layer "F.Cu") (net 4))
 (segment (start 147.5 86.84) (end 158.66 98) (width 1) (layer "F.Cu") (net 5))
 (segment (start 158.66 98) (end 161.5 98) (width 1) (layer "F.Cu") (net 5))
 (segment (start 135.92 103) (end 135.92 102.08) (width 0.2) (layer "F.Cu") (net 1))
 (segment (start 146 83.26) (end 147.5 81.76) (width 0.2) (layer "F.Cu") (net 1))
 (segment (start 134.8 81.76) (end 134.8 84.3) (width 1) (layer "F.Cu") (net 1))
 (segment (start 164 74.5375) (end 165.5 76.0375) (width 0.2) (layer "F.Cu") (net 1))
 (segment (start 170.5 68.4625) (end 168 70.9625) (width 0.2) (layer "F.Cu") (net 1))
 (segment (start 175.88 75.38) (end 172.5 78.76) (width 0.2) (layer "F.Cu") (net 1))
 (segment (start 139 101) (end 141 103) (width 0.2) (layer "F.Cu") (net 1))
 (segment (start 172.5 78.76) (end 172.5 79.5375) (width 0.2) (layer "F.Cu") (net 1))
 (segment (start 140.5 68) (end 132 76.5) (width 1) (layer "F.Cu") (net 1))
 (segment (start 169.5375 81.5375) (end 165.5 77.5) (width 0.2) (layer "F.Cu") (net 1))
 (segment (start 146 95.5) (end 146 83.26) (width 0.2) (layer "F.Cu") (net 1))
 (segment (start 147 97) (end 141 103) (width 0.2) (layer "F.Cu") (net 1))
 (segment (start 168.23 63) (end 168.23 66.1925) (width 0.6) (layer "F.Cu") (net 1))
 (segment (start 165.0375 66.8075) (end 161.23 63) (width 0.6) (layer "F.Cu") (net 1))
 (segment (start 147.5 97) (end 147 97) (width 0.2) (layer "F.Cu") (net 1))
 (segment (start 165.6525 66.1925) (end 165.0375 66.8075) (width 0.6) (layer "F.Cu") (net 1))
 (segment (start 170.0375 86.5) (end 170.0375 82) (width 0.2) (layer "F.Cu") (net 1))
 (segment (start 168.23 66.1925) (end 170.5 68.4625) (width 0.6) (layer "F.Cu") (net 1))
 (segment (start 151.2225 81.76) (end 151.4625 82) (width 0.6) (layer "F.Cu") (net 1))
 (segment (start 166.83063 70.9625) (end 164 73.79313) (width 0.2) (layer "F.Cu") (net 1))
 (segment (start 161.23 63) (end 148.53 63) (width 0.6) (layer "F.Cu") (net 1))
 (segment (start 135.92 102.08) (end 137 101) (width 0.2) (layer "F.Cu") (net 1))
 (segment (start 164 73.79313) (end 164 74.5375) (width 0.2) (layer "F.Cu") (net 1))
 (segment (start 172.5 79.5375) (end 170.5 81.5375) (width 0.2) (layer "F.Cu") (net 1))
 (segment (start 170.0375 82) (end 170.5 81.5375) (width 0.2) (layer "F.Cu") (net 1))
 (segment (start 148.53 63) (end 143.53 68) (width 0.6) (layer "F.Cu") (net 1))
 (segment (start 168 70.9625) (end 166.83063 70.9625) (width 0.2) (layer "F.Cu") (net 1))
 (segment (start 165.0375 68.5) (end 165.0375 66.8075) (width 0.6) (layer "F.Cu") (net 1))
 (segment (start 147.5 97) (end 146 95.5) (width 0.2) (layer "F.Cu") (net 1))
 (segment (start 132 76.5) (end 132 78.96) (width 1) (layer "F.Cu") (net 1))
 (segment (start 147.5 81.76) (end 151.2225 81.76) (width 0.6) (layer "F.Cu") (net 1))
 (segment (start 170.5 81.5375) (end 169.5375 81.5375) (width 0.2) (layer "F.Cu") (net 1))
 (segment (start 155.5 70.42) (end 153.2 72.72) (width 1) (layer "F.Cu") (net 1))
 (segment (start 168.23 66.1925) (end 165.6525 66.1925) (width 0.6) (layer "F.Cu") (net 1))
 (segment (start 165.5 77.5) (end 165.5 76.0375) (width 0.2) (layer "F.Cu") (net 1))
 (segment (start 143.53 68) (end 140.5 68) (width 1) (layer "F.Cu") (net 1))
 (segment (start 137 101) (end 139 101) (width 0.2) (layer "F.Cu") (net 1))
 (segment (start 132 78.96) (end 134.8 81.76) (width 1) (layer "F.Cu") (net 1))
 (segment (start 155.5 67.044888) (end 155.5 70.42) (width 1) (layer "F.Cu") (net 1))
 (segment (start 147 63) (end 143.53 66.47) (width 1) (layer "B.Cu") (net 1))
 (segment (start 155.5 67.044888) (end 154.544888 67.044888) (width 1) (layer "B.Cu") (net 1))
 (segment (start 154.544888 67.044888) (end 150.5 63) (width 1) (layer "B.Cu") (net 1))
 (segment (start 143.53 66.47) (end 143.53 68) (width 1) (layer "B.Cu") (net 1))
 (segment (start 150.5 63) (end 147 63) (width 1) (layer "B.Cu") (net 1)))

